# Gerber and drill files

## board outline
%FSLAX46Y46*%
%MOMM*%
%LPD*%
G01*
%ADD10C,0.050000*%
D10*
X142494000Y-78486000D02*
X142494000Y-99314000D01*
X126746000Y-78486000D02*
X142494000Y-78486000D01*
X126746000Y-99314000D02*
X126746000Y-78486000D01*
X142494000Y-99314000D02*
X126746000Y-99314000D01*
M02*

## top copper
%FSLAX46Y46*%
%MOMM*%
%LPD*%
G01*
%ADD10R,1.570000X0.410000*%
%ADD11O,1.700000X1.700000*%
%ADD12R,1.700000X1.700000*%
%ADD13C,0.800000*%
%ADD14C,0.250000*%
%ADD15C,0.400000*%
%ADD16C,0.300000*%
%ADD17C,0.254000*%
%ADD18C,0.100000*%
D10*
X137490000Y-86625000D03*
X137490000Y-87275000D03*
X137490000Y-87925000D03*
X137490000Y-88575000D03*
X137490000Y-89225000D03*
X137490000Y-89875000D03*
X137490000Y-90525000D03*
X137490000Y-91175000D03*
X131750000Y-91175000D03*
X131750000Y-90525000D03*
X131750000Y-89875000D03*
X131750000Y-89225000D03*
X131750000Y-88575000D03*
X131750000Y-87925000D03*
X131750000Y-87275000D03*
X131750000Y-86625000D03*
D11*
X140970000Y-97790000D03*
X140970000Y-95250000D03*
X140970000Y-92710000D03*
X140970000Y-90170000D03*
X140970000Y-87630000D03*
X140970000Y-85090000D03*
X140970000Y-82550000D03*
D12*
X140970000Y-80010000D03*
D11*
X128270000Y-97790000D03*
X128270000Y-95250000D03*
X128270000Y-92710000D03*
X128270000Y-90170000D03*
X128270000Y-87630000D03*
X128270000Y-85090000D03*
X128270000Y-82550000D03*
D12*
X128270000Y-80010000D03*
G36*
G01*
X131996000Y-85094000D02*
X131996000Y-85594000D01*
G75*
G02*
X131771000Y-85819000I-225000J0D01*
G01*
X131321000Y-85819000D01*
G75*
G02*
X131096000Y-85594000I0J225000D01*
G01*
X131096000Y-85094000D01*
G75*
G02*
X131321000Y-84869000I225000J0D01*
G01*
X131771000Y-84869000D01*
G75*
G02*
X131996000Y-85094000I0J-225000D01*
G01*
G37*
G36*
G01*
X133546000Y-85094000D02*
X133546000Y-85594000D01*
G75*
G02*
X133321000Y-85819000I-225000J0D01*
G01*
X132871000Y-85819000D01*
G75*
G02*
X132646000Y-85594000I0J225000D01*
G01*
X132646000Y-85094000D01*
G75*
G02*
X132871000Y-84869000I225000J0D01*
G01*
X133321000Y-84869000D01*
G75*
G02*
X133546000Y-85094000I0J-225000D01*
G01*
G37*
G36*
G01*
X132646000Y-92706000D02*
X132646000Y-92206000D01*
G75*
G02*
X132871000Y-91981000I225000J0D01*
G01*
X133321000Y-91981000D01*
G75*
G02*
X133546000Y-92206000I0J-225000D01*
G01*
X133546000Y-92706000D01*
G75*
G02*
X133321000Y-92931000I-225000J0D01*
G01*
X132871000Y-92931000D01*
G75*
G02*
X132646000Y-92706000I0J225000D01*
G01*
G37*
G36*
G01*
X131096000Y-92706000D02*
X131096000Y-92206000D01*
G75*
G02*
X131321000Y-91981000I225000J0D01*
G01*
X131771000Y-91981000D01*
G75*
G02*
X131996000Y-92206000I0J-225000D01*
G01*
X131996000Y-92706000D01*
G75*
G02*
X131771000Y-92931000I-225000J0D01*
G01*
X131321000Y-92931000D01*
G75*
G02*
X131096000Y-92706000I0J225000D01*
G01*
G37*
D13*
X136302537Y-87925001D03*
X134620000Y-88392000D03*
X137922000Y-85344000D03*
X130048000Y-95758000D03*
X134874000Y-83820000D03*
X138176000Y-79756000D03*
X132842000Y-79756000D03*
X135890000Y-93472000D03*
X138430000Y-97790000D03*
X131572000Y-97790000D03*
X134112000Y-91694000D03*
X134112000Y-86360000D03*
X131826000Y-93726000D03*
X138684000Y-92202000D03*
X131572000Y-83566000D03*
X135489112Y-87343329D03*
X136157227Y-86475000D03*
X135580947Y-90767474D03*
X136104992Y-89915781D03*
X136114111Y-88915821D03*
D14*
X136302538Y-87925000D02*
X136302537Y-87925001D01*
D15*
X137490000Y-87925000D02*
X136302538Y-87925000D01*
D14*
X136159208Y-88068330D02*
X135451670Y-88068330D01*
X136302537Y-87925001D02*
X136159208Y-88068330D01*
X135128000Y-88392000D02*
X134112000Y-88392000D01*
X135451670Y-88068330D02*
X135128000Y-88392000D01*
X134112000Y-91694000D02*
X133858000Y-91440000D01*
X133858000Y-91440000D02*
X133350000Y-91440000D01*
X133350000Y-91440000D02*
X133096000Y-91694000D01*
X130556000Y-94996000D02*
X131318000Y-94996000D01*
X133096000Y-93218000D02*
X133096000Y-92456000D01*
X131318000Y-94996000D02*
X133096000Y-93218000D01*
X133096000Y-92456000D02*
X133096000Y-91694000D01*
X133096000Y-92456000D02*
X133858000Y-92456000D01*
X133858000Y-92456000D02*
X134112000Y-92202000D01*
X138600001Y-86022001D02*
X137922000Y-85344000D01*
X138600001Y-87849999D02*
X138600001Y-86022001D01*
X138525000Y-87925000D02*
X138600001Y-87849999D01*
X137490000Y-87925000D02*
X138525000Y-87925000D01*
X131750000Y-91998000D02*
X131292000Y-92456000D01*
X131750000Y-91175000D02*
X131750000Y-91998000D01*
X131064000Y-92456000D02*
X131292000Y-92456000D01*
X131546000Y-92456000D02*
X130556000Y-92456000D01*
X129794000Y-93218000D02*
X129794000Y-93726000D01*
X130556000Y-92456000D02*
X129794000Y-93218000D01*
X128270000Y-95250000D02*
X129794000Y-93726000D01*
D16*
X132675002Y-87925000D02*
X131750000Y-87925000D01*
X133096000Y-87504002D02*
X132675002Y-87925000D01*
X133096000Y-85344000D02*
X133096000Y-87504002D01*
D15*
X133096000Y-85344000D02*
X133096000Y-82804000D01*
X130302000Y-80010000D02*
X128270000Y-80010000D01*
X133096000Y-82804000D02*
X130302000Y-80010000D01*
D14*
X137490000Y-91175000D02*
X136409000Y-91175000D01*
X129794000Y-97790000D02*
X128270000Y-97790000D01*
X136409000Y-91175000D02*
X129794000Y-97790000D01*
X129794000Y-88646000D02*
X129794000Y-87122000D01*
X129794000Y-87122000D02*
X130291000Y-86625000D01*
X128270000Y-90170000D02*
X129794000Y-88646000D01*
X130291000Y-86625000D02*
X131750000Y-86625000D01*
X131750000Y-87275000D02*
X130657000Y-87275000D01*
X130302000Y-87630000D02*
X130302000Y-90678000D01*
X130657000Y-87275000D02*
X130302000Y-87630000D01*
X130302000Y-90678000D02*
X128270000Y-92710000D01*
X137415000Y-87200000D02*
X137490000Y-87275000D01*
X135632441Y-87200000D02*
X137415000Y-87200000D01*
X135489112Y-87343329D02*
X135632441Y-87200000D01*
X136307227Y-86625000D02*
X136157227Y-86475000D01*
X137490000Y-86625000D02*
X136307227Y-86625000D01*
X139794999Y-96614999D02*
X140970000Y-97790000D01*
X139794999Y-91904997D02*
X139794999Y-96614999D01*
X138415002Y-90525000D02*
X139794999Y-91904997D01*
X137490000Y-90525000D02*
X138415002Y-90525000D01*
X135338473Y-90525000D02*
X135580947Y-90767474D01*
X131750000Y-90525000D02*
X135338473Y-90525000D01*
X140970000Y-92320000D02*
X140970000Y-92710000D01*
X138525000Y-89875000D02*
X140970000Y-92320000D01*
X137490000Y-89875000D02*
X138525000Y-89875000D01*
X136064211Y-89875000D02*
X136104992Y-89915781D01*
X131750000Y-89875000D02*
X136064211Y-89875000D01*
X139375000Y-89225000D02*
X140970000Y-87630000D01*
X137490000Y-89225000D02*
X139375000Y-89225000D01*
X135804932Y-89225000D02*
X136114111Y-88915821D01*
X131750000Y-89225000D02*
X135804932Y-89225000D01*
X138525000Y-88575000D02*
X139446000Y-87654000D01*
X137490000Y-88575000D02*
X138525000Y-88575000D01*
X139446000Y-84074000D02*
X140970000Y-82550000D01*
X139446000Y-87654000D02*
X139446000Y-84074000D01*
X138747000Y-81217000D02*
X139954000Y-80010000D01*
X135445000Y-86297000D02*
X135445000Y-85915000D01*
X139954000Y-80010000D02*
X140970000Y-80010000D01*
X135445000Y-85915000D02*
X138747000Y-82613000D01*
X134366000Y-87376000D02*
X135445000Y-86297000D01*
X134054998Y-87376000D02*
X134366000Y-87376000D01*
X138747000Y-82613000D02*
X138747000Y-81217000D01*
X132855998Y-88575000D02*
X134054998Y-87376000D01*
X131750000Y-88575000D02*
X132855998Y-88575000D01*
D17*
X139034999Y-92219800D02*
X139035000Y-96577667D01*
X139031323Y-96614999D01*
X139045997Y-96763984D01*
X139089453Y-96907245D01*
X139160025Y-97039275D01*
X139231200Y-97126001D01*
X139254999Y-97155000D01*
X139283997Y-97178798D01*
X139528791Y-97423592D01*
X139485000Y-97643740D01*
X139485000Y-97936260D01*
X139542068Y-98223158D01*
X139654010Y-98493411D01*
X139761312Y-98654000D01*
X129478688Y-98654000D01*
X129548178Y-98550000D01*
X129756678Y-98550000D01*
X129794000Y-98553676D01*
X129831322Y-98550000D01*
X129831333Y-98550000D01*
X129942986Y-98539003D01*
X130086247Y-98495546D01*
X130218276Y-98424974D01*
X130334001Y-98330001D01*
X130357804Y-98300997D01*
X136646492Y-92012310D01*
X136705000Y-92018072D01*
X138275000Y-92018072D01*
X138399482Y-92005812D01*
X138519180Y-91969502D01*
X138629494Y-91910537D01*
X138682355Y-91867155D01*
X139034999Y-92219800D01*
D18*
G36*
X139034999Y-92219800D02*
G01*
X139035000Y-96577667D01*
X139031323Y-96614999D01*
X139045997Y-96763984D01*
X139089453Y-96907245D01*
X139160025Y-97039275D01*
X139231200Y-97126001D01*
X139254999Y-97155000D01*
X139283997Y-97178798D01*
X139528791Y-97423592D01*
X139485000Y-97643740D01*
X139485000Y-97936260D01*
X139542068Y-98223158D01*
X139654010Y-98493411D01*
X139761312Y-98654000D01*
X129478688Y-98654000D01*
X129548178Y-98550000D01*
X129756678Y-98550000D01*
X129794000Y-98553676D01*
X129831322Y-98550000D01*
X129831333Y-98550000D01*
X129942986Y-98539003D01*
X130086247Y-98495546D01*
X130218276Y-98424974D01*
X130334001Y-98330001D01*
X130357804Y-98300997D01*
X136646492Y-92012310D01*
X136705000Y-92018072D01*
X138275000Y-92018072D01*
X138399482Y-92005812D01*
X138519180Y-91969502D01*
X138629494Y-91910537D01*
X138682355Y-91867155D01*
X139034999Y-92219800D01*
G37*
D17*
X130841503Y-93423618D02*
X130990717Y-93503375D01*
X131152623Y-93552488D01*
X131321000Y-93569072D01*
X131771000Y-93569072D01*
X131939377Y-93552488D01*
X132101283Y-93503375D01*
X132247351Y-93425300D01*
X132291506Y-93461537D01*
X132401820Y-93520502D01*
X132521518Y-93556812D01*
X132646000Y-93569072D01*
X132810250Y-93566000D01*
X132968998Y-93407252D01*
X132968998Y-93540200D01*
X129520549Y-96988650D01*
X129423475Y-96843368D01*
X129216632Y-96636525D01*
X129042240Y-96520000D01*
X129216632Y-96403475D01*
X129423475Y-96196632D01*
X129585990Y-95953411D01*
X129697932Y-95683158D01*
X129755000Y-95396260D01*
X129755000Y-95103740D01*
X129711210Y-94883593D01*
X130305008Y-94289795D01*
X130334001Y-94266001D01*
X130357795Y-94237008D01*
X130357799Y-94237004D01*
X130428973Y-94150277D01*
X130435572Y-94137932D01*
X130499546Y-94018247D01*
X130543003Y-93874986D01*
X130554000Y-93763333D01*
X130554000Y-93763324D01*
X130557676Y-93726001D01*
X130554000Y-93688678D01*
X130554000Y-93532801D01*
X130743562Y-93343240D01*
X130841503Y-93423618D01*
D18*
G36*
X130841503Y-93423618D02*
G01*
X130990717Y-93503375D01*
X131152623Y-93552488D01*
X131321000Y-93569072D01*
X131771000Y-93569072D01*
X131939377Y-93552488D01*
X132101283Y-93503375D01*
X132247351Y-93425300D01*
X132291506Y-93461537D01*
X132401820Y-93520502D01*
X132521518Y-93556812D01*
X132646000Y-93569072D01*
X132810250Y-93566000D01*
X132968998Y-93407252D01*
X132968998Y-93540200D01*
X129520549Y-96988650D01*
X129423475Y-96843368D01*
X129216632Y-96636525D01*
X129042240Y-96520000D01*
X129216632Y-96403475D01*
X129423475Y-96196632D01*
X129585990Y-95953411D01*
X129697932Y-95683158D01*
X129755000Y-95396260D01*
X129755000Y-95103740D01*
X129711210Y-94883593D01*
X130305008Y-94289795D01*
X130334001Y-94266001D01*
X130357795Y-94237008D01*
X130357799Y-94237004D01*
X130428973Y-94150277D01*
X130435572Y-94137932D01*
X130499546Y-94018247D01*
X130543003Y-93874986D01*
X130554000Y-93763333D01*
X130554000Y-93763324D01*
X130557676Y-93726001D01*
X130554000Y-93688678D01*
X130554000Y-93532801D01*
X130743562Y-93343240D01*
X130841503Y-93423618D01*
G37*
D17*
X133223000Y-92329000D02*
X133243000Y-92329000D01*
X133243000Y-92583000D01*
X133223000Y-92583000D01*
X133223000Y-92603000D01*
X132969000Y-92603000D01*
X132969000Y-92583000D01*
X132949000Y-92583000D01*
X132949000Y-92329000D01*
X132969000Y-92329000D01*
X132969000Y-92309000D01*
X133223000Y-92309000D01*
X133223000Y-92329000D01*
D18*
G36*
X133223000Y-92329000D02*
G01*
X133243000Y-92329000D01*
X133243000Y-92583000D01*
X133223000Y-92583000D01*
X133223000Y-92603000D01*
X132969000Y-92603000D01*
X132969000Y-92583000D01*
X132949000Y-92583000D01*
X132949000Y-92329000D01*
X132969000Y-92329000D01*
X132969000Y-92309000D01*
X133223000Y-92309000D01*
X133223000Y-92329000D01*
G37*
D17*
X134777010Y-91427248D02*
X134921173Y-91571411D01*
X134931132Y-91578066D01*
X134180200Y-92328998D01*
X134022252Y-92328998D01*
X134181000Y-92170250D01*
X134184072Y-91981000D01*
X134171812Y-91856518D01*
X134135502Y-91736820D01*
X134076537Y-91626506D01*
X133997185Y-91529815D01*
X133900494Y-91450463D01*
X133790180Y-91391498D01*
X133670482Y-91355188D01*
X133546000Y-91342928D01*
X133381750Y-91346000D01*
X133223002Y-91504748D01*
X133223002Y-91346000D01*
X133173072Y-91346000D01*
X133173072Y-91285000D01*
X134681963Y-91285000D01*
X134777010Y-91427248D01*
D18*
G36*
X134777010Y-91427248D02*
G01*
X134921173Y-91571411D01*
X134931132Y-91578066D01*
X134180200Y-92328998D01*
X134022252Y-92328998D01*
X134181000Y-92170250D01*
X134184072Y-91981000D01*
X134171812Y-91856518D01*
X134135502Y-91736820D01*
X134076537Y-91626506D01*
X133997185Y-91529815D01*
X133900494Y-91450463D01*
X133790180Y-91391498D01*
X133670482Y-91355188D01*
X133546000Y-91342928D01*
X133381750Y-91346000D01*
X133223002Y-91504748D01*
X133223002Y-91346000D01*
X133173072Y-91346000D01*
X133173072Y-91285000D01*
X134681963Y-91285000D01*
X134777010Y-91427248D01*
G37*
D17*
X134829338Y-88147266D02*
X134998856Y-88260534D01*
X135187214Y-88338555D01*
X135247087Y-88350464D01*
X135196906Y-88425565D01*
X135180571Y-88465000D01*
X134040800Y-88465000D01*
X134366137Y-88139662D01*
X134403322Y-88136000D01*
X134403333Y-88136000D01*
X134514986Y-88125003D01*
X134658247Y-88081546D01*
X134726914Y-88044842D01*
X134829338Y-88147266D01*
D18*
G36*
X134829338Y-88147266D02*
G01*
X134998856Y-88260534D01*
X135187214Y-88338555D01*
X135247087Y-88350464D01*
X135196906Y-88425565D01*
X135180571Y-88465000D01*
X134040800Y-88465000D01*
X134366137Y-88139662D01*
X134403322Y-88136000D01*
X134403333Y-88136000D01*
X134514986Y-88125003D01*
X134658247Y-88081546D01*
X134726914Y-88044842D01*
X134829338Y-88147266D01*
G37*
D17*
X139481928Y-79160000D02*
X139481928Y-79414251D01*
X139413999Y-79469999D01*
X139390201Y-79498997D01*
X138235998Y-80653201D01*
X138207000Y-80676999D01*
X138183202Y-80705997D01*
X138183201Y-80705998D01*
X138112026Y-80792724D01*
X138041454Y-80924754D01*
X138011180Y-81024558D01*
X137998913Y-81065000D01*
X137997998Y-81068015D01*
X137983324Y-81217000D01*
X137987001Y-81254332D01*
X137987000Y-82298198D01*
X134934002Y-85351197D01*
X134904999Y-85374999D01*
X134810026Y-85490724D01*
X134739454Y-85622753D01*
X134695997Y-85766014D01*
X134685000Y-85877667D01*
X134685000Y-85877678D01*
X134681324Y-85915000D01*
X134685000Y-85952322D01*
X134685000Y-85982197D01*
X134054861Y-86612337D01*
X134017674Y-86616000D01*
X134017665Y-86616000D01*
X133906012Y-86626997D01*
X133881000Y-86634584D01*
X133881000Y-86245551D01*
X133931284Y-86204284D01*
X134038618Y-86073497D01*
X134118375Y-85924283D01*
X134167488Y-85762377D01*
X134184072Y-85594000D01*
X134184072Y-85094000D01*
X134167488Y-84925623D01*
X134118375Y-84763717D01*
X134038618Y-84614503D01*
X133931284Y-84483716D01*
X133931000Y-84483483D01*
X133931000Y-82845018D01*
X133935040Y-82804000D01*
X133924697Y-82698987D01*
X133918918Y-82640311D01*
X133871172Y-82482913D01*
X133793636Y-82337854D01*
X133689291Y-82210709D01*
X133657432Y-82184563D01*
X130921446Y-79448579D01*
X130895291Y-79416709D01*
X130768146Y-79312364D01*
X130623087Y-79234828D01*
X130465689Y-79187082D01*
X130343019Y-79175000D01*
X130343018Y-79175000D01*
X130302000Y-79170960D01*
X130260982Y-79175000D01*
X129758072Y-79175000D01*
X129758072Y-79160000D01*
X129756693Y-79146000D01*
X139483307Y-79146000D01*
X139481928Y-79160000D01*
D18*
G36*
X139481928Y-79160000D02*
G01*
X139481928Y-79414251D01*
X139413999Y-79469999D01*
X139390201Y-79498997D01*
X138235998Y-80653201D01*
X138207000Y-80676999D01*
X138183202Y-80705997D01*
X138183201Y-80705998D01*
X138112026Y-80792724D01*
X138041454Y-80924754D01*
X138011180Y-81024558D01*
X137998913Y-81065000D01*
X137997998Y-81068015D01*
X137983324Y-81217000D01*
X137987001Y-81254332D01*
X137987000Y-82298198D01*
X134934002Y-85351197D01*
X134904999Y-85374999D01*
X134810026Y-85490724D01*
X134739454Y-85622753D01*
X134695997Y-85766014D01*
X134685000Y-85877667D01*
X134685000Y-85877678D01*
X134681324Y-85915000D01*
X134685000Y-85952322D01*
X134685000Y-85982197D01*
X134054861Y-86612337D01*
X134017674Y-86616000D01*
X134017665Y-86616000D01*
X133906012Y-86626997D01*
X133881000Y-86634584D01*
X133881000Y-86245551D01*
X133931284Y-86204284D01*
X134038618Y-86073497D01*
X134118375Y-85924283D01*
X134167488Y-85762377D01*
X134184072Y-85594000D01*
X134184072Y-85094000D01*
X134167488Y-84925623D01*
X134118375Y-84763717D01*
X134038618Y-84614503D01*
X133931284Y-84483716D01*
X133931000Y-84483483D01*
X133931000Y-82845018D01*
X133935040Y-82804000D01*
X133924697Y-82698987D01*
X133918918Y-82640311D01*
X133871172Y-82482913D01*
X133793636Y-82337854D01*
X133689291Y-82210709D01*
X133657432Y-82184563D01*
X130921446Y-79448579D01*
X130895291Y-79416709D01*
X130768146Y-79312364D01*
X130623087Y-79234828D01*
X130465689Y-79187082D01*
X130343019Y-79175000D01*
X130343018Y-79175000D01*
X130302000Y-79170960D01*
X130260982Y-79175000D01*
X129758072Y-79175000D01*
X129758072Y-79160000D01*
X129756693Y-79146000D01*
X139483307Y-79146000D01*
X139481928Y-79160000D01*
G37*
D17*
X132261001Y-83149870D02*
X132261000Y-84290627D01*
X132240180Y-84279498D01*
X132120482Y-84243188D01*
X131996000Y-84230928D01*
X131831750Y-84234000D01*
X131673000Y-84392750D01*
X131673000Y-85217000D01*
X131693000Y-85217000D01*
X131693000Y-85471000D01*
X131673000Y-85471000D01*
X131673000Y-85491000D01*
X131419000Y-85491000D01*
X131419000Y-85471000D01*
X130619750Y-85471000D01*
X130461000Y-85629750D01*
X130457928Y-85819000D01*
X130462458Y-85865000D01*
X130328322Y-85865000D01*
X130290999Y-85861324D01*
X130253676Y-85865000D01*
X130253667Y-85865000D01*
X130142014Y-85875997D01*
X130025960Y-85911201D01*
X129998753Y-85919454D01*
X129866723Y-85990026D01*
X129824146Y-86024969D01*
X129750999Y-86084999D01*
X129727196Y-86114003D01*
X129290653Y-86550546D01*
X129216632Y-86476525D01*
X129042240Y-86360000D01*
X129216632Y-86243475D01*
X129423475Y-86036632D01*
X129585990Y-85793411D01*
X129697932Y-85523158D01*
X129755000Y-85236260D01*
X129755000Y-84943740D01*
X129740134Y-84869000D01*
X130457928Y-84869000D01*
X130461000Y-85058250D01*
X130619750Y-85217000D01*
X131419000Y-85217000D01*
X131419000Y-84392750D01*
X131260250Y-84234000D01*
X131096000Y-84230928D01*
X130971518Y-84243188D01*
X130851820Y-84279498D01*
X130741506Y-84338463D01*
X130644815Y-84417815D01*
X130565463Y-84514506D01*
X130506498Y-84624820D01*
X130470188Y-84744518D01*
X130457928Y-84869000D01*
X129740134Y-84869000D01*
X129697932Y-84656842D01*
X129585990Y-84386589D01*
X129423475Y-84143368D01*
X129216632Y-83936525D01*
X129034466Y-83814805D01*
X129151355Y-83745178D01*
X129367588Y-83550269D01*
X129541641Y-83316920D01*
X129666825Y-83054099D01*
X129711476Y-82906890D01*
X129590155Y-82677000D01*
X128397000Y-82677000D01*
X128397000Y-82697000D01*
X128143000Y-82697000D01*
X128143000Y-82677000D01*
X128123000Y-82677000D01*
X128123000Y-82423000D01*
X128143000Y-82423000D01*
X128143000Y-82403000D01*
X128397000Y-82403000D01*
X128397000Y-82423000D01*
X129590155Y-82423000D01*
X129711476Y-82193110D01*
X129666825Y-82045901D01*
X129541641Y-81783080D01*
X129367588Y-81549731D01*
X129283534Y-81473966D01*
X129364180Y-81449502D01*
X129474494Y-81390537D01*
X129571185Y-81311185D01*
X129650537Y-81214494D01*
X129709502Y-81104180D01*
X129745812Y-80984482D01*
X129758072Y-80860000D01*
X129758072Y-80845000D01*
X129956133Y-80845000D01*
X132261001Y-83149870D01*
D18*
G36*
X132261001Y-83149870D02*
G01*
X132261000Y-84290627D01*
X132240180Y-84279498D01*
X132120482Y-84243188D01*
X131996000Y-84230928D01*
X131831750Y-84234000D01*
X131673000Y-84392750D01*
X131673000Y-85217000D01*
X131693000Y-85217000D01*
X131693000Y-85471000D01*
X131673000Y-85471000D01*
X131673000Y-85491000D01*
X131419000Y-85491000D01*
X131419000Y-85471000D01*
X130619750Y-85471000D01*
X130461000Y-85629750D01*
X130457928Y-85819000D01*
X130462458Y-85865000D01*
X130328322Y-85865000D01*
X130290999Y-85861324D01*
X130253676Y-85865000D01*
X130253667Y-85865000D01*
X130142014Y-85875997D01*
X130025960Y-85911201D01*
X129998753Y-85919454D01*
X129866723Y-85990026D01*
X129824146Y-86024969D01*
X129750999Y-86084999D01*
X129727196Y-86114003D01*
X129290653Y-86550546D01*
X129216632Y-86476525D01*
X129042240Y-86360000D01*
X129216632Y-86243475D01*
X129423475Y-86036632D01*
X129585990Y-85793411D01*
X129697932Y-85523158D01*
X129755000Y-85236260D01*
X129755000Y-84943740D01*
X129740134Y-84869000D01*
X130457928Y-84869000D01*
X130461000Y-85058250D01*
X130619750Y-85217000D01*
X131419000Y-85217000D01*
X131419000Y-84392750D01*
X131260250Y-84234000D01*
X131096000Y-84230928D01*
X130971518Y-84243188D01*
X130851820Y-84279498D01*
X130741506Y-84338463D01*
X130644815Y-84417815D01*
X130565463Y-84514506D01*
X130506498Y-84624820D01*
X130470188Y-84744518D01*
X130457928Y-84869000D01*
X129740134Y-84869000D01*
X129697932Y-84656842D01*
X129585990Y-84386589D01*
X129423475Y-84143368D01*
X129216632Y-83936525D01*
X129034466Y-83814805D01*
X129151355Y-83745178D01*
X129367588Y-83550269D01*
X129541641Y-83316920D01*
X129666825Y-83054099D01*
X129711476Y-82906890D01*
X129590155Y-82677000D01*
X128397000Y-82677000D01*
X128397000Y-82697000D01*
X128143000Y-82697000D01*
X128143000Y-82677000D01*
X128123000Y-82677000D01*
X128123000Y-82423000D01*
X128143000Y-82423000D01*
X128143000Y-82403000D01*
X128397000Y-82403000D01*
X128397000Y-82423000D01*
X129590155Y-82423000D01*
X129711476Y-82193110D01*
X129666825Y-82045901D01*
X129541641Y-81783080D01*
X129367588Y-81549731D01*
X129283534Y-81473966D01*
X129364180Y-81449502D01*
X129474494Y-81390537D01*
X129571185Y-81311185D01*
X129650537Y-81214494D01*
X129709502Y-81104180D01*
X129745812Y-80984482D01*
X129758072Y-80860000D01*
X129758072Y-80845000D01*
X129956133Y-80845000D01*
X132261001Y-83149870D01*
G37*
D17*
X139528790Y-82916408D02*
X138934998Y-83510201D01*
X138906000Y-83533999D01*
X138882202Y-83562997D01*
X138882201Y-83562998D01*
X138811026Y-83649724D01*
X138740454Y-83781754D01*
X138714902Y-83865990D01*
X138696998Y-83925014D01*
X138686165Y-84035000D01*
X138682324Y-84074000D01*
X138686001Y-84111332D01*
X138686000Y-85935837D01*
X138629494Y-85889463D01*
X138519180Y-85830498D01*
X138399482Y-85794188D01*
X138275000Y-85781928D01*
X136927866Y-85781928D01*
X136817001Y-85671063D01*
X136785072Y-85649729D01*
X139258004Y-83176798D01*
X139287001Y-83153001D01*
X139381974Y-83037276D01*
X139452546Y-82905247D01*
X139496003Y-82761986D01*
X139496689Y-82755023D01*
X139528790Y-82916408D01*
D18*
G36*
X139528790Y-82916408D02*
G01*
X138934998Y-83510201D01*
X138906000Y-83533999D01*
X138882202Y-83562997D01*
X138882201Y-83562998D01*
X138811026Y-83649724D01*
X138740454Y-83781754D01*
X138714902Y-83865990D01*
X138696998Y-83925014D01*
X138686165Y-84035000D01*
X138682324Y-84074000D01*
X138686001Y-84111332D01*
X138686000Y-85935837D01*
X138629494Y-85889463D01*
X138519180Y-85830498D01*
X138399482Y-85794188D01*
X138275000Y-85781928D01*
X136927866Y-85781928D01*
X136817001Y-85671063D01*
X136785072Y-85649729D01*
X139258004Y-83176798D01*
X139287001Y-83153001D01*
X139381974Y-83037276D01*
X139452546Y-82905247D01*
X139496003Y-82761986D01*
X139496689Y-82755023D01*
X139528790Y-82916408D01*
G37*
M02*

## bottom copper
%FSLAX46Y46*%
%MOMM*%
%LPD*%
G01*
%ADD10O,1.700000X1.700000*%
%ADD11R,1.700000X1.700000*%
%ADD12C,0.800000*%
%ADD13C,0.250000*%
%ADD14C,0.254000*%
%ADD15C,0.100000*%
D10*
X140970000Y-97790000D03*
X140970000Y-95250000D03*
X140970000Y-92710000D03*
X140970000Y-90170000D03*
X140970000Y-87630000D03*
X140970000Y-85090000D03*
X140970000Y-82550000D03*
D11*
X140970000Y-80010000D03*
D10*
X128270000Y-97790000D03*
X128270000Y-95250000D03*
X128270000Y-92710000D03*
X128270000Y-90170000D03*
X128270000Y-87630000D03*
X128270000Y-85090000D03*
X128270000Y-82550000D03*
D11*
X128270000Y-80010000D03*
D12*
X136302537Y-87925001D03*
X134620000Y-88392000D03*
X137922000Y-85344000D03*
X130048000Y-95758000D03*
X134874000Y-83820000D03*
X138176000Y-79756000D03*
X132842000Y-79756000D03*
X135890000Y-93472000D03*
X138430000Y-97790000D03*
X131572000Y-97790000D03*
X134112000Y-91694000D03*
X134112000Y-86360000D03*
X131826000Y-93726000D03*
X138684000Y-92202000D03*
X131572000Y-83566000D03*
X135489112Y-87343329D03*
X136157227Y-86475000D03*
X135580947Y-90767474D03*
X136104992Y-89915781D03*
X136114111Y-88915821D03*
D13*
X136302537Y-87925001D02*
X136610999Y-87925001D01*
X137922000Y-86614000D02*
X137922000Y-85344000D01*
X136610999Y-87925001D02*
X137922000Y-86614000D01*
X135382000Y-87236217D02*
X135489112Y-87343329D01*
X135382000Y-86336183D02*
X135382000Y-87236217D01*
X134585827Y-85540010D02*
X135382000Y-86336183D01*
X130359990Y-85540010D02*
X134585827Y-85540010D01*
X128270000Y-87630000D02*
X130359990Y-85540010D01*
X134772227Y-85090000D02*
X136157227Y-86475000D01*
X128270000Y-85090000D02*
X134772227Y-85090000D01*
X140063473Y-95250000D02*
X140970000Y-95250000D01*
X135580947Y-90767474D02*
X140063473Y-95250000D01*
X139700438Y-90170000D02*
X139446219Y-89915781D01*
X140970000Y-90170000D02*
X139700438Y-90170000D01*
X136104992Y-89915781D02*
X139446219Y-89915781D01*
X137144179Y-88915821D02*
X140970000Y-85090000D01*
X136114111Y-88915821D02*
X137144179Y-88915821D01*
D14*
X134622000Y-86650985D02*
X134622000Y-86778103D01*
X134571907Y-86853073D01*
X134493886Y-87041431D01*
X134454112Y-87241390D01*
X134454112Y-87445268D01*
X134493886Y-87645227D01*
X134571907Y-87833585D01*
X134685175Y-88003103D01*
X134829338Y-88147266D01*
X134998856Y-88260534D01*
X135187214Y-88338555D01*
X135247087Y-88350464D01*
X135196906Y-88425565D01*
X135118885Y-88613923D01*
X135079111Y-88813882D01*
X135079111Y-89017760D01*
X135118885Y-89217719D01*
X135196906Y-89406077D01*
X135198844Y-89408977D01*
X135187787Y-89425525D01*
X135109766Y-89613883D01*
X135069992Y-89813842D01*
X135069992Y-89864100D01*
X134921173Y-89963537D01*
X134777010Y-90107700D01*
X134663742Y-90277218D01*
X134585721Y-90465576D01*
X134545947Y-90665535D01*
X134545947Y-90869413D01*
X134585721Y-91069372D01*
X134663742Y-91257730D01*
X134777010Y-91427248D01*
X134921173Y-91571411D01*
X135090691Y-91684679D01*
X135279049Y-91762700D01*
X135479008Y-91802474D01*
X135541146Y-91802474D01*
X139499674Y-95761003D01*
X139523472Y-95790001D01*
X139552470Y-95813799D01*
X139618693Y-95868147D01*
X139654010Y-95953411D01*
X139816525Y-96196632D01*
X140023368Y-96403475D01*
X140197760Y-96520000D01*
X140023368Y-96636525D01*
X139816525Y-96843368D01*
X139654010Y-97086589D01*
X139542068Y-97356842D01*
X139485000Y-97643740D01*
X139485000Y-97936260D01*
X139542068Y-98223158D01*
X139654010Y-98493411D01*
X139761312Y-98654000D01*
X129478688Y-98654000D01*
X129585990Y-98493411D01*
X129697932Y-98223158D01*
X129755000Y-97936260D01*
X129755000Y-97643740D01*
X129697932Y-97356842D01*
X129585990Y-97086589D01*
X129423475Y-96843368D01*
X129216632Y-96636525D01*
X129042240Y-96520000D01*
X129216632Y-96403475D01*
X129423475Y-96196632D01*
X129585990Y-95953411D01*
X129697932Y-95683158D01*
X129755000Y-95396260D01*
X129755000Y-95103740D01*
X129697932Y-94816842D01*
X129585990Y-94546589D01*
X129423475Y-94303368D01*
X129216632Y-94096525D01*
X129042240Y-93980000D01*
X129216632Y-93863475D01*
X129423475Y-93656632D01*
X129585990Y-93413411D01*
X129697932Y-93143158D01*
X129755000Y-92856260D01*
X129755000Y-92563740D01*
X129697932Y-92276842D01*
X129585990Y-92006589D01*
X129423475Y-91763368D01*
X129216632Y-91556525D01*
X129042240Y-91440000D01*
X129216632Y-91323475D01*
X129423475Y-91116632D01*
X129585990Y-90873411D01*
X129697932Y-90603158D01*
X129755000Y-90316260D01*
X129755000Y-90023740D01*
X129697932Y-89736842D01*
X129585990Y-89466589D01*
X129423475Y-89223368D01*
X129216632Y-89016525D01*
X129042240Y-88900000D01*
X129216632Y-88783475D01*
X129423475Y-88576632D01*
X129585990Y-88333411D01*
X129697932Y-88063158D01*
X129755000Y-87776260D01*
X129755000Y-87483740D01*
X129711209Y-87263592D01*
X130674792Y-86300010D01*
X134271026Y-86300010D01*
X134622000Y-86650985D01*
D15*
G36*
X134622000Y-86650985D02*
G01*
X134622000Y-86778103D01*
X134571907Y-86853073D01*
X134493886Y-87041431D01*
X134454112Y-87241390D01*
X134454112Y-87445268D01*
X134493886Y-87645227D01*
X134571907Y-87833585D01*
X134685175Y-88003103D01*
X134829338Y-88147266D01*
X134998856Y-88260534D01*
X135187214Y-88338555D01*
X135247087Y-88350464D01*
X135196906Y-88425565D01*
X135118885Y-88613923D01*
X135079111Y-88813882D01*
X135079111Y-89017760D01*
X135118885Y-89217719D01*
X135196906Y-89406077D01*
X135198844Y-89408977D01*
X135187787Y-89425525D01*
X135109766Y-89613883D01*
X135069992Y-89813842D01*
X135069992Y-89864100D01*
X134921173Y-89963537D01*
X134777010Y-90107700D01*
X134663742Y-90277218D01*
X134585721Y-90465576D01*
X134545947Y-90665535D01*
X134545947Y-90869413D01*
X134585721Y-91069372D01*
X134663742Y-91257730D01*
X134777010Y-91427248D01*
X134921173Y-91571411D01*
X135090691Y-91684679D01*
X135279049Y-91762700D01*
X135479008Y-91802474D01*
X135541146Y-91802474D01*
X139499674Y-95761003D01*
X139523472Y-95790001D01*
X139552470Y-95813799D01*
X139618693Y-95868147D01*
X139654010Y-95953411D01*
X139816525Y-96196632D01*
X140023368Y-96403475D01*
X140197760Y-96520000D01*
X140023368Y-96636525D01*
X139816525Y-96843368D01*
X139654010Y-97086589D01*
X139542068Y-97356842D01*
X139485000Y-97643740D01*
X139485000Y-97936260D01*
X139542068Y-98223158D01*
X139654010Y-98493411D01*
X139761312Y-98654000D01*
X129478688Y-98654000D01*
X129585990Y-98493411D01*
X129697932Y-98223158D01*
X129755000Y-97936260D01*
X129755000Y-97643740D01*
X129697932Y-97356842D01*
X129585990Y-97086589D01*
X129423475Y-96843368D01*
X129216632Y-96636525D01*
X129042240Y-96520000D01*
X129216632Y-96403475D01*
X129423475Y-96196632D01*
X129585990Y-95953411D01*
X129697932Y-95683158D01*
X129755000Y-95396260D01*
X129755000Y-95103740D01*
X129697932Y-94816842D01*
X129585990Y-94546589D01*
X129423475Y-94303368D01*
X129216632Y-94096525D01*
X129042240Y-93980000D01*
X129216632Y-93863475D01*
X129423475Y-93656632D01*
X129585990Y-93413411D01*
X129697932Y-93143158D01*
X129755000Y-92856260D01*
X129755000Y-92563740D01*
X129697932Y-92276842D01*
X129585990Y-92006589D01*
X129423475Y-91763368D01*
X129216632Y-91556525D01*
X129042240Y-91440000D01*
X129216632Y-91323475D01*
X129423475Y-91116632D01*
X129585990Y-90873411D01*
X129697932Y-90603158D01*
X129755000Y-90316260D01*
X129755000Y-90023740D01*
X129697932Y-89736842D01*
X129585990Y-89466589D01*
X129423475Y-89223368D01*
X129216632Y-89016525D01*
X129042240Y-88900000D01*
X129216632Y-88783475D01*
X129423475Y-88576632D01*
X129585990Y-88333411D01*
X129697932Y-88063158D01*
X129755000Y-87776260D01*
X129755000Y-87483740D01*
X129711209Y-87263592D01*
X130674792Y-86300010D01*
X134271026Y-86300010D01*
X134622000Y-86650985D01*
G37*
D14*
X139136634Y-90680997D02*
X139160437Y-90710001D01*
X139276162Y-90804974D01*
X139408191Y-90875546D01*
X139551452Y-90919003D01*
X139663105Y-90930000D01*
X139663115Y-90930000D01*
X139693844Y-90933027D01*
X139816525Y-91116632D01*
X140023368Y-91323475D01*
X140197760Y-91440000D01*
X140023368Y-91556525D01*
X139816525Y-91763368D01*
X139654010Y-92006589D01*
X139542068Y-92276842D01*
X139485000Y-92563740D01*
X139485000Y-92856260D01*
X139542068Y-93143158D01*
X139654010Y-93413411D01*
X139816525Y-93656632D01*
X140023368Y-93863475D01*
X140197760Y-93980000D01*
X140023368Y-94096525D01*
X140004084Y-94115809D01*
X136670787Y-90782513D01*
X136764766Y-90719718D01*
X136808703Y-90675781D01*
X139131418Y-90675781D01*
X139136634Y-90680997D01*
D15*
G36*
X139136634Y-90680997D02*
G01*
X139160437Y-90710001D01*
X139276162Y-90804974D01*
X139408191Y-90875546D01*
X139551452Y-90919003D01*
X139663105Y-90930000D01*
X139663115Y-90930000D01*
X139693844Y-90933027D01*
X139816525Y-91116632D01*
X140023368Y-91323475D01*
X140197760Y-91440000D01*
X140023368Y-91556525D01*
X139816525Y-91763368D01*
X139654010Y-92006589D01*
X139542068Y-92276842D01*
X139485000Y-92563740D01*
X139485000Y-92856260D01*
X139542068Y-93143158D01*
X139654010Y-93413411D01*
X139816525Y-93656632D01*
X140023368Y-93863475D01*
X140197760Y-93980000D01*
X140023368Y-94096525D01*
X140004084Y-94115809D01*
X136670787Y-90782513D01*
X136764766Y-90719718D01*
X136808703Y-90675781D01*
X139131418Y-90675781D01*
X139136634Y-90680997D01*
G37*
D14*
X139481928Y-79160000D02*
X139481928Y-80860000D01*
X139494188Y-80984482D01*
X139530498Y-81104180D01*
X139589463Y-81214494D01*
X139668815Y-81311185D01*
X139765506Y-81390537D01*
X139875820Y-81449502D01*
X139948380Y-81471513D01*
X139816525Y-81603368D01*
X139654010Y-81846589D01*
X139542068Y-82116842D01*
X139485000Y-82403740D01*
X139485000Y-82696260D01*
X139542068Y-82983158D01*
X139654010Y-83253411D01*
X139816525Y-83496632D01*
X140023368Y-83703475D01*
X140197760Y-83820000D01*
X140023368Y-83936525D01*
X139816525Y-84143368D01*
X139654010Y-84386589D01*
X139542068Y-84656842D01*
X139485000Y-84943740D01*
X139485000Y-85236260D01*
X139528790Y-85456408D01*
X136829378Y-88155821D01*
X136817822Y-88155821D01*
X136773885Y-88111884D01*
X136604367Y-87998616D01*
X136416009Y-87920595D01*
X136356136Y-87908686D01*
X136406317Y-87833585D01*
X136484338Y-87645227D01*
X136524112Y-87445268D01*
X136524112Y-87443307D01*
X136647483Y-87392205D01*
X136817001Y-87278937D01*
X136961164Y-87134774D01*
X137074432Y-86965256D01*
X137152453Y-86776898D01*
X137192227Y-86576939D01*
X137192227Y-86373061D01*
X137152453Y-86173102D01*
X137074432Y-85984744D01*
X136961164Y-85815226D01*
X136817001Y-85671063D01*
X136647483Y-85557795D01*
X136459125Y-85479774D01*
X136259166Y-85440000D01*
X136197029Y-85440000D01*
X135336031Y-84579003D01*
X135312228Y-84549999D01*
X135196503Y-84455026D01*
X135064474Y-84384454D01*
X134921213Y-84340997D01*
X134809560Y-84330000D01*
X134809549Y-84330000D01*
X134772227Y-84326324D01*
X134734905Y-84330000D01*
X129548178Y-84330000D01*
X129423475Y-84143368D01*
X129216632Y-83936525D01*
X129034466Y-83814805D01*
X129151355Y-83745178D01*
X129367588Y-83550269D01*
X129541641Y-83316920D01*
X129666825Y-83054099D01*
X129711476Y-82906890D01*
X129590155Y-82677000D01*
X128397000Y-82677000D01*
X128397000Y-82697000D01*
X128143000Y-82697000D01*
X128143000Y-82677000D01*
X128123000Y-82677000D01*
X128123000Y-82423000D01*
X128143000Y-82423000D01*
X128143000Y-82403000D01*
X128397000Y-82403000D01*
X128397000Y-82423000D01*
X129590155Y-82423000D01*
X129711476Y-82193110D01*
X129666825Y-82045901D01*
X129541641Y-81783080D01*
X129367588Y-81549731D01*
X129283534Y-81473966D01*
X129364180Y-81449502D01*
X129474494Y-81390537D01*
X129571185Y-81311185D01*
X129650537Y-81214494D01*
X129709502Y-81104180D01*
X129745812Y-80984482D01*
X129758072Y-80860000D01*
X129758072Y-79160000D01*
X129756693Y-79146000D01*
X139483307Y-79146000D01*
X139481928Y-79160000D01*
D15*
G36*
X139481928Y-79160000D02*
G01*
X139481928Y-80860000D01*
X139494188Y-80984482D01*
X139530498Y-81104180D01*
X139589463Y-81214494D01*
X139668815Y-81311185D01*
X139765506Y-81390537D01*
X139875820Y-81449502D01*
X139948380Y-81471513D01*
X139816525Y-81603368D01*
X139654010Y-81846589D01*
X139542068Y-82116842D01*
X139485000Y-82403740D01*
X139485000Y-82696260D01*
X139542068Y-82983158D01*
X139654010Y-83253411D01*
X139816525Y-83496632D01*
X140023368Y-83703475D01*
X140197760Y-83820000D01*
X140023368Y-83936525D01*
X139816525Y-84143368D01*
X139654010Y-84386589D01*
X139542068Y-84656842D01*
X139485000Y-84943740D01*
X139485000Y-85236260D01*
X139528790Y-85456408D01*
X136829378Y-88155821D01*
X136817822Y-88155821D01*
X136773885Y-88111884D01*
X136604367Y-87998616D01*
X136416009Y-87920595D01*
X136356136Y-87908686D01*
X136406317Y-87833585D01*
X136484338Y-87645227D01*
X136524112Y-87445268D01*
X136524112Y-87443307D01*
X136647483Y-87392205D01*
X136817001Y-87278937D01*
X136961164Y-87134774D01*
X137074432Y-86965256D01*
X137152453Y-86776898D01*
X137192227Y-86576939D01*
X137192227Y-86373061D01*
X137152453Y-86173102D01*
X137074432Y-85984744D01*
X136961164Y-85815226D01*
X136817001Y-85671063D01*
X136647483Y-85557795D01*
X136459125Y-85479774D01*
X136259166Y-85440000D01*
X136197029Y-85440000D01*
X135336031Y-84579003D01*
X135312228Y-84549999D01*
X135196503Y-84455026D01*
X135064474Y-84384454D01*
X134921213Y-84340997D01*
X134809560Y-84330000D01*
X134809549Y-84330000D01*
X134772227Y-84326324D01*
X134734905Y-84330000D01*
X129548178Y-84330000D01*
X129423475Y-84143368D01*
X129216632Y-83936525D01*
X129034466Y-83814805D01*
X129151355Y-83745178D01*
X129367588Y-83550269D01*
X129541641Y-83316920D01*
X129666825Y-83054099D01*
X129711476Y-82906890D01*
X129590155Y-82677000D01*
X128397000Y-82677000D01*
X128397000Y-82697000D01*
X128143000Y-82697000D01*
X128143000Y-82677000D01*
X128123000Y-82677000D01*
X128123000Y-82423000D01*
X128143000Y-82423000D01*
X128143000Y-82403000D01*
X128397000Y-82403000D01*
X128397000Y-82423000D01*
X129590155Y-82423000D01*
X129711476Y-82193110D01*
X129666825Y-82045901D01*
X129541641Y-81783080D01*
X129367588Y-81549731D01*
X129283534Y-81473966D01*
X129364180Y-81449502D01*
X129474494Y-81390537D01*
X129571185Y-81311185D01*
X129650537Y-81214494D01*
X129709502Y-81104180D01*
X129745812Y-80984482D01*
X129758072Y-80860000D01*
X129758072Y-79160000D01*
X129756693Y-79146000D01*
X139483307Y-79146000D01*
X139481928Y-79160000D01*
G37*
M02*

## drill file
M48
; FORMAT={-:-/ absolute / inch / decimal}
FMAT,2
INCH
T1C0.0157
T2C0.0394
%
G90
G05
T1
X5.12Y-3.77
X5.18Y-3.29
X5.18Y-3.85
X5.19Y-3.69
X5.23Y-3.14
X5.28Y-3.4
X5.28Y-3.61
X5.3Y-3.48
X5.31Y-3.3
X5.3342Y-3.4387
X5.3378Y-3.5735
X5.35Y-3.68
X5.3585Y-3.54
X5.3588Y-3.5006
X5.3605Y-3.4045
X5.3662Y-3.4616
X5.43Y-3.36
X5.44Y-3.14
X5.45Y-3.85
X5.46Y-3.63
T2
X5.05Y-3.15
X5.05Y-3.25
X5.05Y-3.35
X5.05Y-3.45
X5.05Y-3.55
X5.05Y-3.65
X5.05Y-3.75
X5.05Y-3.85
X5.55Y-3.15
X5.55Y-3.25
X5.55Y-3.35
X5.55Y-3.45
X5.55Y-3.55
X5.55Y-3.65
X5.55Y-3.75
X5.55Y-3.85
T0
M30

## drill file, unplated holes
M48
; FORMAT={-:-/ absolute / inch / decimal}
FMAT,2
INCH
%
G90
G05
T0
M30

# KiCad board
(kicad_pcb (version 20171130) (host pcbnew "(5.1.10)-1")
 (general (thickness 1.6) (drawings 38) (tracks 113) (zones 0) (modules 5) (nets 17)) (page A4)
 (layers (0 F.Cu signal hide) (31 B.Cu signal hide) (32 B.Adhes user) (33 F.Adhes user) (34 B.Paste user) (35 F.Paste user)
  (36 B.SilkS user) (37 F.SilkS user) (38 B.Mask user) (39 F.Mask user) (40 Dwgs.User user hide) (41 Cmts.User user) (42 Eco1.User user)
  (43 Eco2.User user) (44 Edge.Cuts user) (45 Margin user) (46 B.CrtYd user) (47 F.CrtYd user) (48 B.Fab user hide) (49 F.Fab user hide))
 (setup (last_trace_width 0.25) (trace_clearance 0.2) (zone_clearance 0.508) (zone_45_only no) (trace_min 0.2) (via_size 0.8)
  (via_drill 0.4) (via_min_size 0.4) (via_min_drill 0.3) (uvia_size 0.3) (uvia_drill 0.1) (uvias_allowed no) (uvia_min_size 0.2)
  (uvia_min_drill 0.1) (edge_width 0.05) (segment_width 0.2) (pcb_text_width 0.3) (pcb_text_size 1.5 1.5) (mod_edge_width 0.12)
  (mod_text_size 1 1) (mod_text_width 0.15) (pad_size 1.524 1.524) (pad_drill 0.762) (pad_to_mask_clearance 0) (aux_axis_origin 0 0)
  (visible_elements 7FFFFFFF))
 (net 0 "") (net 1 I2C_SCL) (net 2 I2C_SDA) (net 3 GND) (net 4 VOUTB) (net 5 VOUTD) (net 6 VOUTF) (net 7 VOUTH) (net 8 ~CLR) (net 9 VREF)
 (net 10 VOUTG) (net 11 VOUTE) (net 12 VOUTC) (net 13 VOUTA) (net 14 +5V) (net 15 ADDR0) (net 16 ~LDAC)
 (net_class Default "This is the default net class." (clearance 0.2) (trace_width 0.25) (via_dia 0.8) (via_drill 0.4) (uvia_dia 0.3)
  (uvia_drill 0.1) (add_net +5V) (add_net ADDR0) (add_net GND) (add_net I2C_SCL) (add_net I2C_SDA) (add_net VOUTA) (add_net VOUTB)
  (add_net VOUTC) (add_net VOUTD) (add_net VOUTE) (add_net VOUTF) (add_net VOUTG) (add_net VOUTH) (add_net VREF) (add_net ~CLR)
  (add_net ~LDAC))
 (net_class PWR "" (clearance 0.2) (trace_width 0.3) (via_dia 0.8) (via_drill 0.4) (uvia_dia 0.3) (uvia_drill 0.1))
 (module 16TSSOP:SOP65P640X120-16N (layer F.Cu) (at 134.62 88.9)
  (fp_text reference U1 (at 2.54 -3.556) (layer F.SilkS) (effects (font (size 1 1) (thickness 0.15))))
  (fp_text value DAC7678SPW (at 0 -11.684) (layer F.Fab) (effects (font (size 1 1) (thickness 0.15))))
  (pad 16 smd rect (at 2.87 -2.275) (size 1.57 0.41) (layers F.Cu F.Paste F.Mask) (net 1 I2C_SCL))
  (pad 15 smd rect (at 2.87 -1.625) (size 1.57 0.41) (layers F.Cu F.Paste F.Mask) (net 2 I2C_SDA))
  (pad 14 smd rect (at 2.87 -0.975) (size 1.57 0.41) (layers F.Cu F.Paste F.Mask) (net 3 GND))
  (pad 13 smd rect (at 2.87 -0.325) (size 1.57 0.41) (layers F.Cu F.Paste F.Mask) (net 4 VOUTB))
  (pad 12 smd rect (at 2.87 0.325) (size 1.57 0.41) (layers F.Cu F.Paste F.Mask) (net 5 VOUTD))
  (pad 11 smd rect (at 2.87 0.975) (size 1.57 0.41) (layers F.Cu F.Paste F.Mask) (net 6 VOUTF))
  (pad 10 smd rect (at 2.87 1.625) (size 1.57 0.41) (layers F.Cu F.Paste F.Mask) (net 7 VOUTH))
  (pad 9 smd rect (at 2.87 2.275) (size 1.57 0.41) (layers F.Cu F.Paste F.Mask) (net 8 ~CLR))
  (pad 8 smd rect (at -2.87 2.275) (size 1.57 0.41) (layers F.Cu F.Paste F.Mask) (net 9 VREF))
  (pad 7 smd rect (at -2.87 1.625) (size 1.57 0.41) (layers F.Cu F.Paste F.Mask) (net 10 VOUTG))
  (pad 6 smd rect (at -2.87 0.975) (size 1.57 0.41) (layers F.Cu F.Paste F.Mask) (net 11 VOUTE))
  (pad 5 smd rect (at -2.87 0.325) (size 1.57 0.41) (layers F.Cu F.Paste F.Mask) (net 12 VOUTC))
  (pad 4 smd rect (at -2.87 -0.325) (size 1.57 0.41) (layers F.Cu F.Paste F.Mask) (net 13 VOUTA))
  (pad 3 smd rect (at -2.87 -0.975) (size 1.57 0.41) (layers F.Cu F.Paste F.Mask) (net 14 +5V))
  (pad 2 smd rect (at -2.87 -1.625) (size 1.57 0.41) (layers F.Cu F.Paste F.Mask) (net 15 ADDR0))
  (pad 1 smd rect (at -2.87 -2.275) (size 1.57 0.41) (layers F.Cu F.Paste F.Mask) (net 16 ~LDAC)))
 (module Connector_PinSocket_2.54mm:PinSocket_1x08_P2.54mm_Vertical (layer B.Cu) (at 140.97 80.01 180)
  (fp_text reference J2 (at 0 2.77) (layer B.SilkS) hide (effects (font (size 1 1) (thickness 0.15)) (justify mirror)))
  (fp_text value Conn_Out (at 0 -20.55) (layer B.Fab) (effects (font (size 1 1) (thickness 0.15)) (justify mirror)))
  (pad 8 thru_hole oval (at 0 -17.78 180) (size 1.7 1.7) (drill 1) (layers *.Cu *.Mask) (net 7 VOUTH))
  (pad 7 thru_hole oval (at 0 -15.24 180) (size 1.7 1.7) (drill 1) (layers *.Cu *.Mask) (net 10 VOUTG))
  (pad 6 thru_hole oval (at 0 -12.7 180) (size 1.7 1.7) (drill 1) (layers *.Cu *.Mask) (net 6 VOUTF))
  (pad 5 thru_hole oval (at 0 -10.16 180) (size 1.7 1.7) (drill 1) (layers *.Cu *.Mask) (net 11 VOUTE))
  (pad 4 thru_hole oval (at 0 -7.62 180) (size 1.7 1.7) (drill 1) (layers *.Cu *.Mask) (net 5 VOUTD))
  (pad 3 thru_hole oval (at 0 -5.08 180) (size 1.7 1.7) (drill 1) (layers *.Cu *.Mask) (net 12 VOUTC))
  (pad 2 thru_hole oval (at 0 -2.54 180) (size 1.7 1.7) (drill 1) (layers *.Cu *.Mask) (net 4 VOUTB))
  (pad 1 thru_hole rect (at 0 0 180) (size 1.7 1.7) (drill 1) (layers *.Cu *.Mask) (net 13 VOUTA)))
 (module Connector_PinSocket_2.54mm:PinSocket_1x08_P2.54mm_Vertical (layer B.Cu) (at 128.27 80.01 180)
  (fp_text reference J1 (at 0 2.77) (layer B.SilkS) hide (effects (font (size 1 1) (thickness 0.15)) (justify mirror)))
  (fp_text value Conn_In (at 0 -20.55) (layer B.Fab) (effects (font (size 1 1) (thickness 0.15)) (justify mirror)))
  (pad 8 thru_hole oval (at 0 -17.78 180) (size 1.7 1.7) (drill 1) (layers *.Cu *.Mask) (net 8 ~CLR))
  (pad 7 thru_hole oval (at 0 -15.24 180) (size 1.7 1.7) (drill 1) (layers *.Cu *.Mask) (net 9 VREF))
  (pad 6 thru_hole oval (at 0 -12.7 180) (size 1.7 1.7) (drill 1) (layers *.Cu *.Mask) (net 15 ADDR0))
  (pad 5 thru_hole oval (at 0 -10.16 180) (size 1.7 1.7) (drill 1) (layers *.Cu *.Mask) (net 16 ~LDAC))
  (pad 4 thru_hole oval (at 0 -7.62 180) (size 1.7 1.7) (drill 1) (layers *.Cu *.Mask) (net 2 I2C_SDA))
  (pad 3 thru_hole oval (at 0 -5.08 180) (size 1.7 1.7) (drill 1) (layers *.Cu *.Mask) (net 1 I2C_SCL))
  (pad 2 thru_hole oval (at 0 -2.54 180) (size 1.7 1.7) (drill 1) (layers *.Cu *.Mask) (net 3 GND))
  (pad 1 thru_hole rect (at 0 0 180) (size 1.7 1.7) (drill 1) (layers *.Cu *.Mask) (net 14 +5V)))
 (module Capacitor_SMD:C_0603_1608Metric (layer F.Cu) (at 132.321 85.344 180)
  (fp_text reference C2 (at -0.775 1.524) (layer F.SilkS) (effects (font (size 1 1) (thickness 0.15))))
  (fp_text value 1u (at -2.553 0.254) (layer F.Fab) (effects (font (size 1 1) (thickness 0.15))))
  (pad 2 smd roundrect (at 0.775 0 180) (size 0.9 0.95) (layers F.Cu F.Paste F.Mask) (roundrect_rratio 0.25) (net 3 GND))
  (pad 1 smd roundrect (at -0.775 0 180) (size 0.9 0.95) (layers F.Cu F.Paste F.Mask) (roundrect_rratio 0.25) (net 14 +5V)))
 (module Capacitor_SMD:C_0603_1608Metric (layer F.Cu) (at 132.321 92.456)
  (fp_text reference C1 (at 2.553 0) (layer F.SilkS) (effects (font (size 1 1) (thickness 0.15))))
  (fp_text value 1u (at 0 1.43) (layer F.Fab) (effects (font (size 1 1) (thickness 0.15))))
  (pad 2 smd roundrect (at 0.775 0) (size 0.9 0.95) (layers F.Cu F.Paste F.Mask) (roundrect_rratio 0.25) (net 3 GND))
  (pad 1 smd roundrect (at -0.775 0) (size 0.9 0.95) (layers F.Cu F.Paste F.Mask) (roundrect_rratio 0.25) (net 9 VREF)))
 (gr_line (start 142.494 78.486) (end 142.494 99.314) (layer Edge.Cuts) (width 0.05))
 (gr_line (start 126.746 78.486) (end 142.494 78.486) (layer Edge.Cuts) (width 0.05))
 (gr_line (start 126.746 99.314) (end 126.746 78.486) (layer Edge.Cuts) (width 0.05))
 (gr_line (start 142.494 99.314) (end 126.746 99.314) (layer Edge.Cuts) (width 0.05))
 (via (at 136.302537 87.925001) (size 0.8) (drill 0.4) (layers F.Cu B.Cu) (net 3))
 (segment (start 136.302538 87.925) (end 136.302537 87.925001) (width 0.25) (layer F.Cu) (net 3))
 (segment (start 137.49 87.925) (end 136.302538 87.925) (width 0.4) (layer F.Cu) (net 3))
 (via (at 134.62 88.392) (size 0.8) (drill 0.4) (layers F.Cu B.Cu) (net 3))
 (segment (start 136.159208 88.06833) (end 135.45167 88.06833) (width 0.25) (layer F.Cu) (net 3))
 (segment (start 136.302537 87.925001) (end 136.159208 88.06833) (width 0.25) (layer F.Cu) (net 3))
 (segment (start 135.128 88.392) (end 134.112 88.392) (width 0.25) (layer F.Cu) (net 3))
 (segment (start 135.45167 88.06833) (end 135.128 88.392) (width 0.25) (layer F.Cu) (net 3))
 (segment (start 136.302537 87.925001) (end 136.610999 87.925001) (width 0.25) (layer B.Cu) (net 3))
 (via (at 137.922 85.344) (size 0.8) (drill 0.4) (layers F.Cu B.Cu) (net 3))
 (segment (start 137.922 86.614) (end 137.922 85.344) (width 0.25) (layer B.Cu) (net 3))
 (segment (start 136.610999 87.925001) (end 137.922 86.614) (width 0.25) (layer B.Cu) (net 3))
 (via (at 130.048 95.758) (size 0.8) (drill 0.4) (layers F.Cu B.Cu) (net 3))
 (via (at 134.874 83.82) (size 0.8) (drill 0.4) (layers F.Cu B.Cu) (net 3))
 (via (at 138.176 79.756) (size 0.8) (drill 0.4) (layers F.Cu B.Cu) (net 3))
 (via (at 132.842 79.756) (size 0.8) (drill 0.4) (layers F.Cu B.Cu) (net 3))
 (via (at 135.89 93.472) (size 0.8) (drill 0.4) (layers F.Cu B.Cu) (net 3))
 (via (at 138.43 97.79) (size 0.8) (drill 0.4) (layers F.Cu B.Cu) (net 3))
 (via (at 131.572 97.79) (size 0.8) (drill 0.4) (layers F.Cu B.Cu) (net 3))
 (via (at 134.112 91.694) (size 0.8) (drill 0.4) (layers F.Cu B.Cu) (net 3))
 (via (at 134.112 86.36) (size 0.8) (drill 0.4) (layers F.Cu B.Cu) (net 3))
 (segment (start 134.112 91.694) (end 133.858 91.44) (width 0.25) (layer F.Cu) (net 3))
 (segment (start 133.858 91.44) (end 133.35 91.44) (width 0.25) (layer F.Cu) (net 3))
 (segment (start 133.35 91.44) (end 133.096 91.694) (width 0.25) (layer F.Cu) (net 3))
 (segment (start 130.556 94.996) (end 131.318 94.996) (width 0.25) (layer F.Cu) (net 3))
 (segment (start 133.096 93.218) (end 133.096 92.456) (width 0.25) (layer F.Cu) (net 3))
 (segment (start 131.318 94.996) (end 133.096 93.218) (width 0.25) (layer F.Cu) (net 3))
 (segment (start 133.096 92.456) (end 133.096 91.694) (width 0.25) (layer F.Cu) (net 3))
 (segment (start 133.096 92.456) (end 133.858 92.456) (width 0.25) (layer F.Cu) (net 3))
 (segment (start 133.858 92.456) (end 134.112 92.202) (width 0.25) (layer F.Cu) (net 3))
 (via (at 131.826 93.726) (size 0.8) (drill 0.4) (layers F.Cu B.Cu) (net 3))
 (via (at 138.684 92.202) (size 0.8) (drill 0.4) (layers F.Cu B.Cu) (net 3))
 (segment (start 138.600001 86.022001) (end 137.922 85.344) (width 0.25) (layer F.Cu) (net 3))
 (segment (start 138.600001 87.849999) (end 138.600001 86.022001) (width 0.25) (layer F.Cu) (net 3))
 (segment (start 138.525 87.925) (end 138.600001 87.849999) (width 0.25) (layer F.Cu) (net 3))
 (segment (start 137.49 87.925) (end 138.525 87.925) (width 0.25) (layer F.Cu) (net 3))
 (via (at 131.572 83.566) (size 0.8) (drill 0.4) (layers F.Cu B.Cu) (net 3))
 (segment (start 131.75 91.998) (end 131.292 92.456) (width 0.25) (layer F.Cu) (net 9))
 (segment (start 131.75 91.175) (end 131.75 91.998) (width 0.25) (layer F.Cu) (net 9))
 (segment (start 131.064 92.456) (end 131.292 92.456) (width 0.25) (layer F.Cu) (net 9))
 (segment (start 131.546 92.456) (end 130.556 92.456) (width 0.25) (layer F.Cu) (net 9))
 (segment (start 129.794 93.218) (end 129.794 93.726) (width 0.25) (layer F.Cu) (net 9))
 (segment (start 130.556 92.456) (end 129.794 93.218) (width 0.25) (layer F.Cu) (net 9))
 (segment (start 128.27 95.25) (end 129.794 93.726) (width 0.25) (layer F.Cu) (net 9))
 (segment (start 132.675002 87.925) (end 131.75 87.925) (width 0.3) (layer F.Cu) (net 14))
 (segment (start 133.096 87.504002) (end 132.675002 87.925) (width 0.3) (layer F.Cu) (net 14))
 (segment (start 133.096 85.344) (end 133.096 87.504002) (width 0.3) (layer F.Cu) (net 14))
 (segment (start 133.096 85.344) (end 133.096 82.804) (width 0.4) (layer F.Cu) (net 14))
 (segment (start 130.302 80.01) (end 128.27 80.01) (width 0.4) (layer F.Cu) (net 14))
 (segment (start 133.096 82.804) (end 130.302 80.01) (width 0.4) (layer F.Cu) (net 14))
 (segment (start 137.49 91.175) (end 136.409 91.175) (width 0.25) (layer F.Cu) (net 8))
 (segment (start 129.794 97.79) (end 128.27 97.79) (width 0.25) (layer F.Cu) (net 8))
 (segment (start 136.409 91.175) (end 129.794 97.79) (width 0.25) (layer F.Cu) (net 8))
 (segment (start 129.794 88.646) (end 129.794 87.122) (width 0.25) (layer F.Cu) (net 16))
 (segment (start 129.794 87.122) (end 130.291 86.625) (width 0.25) (layer F.Cu) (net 16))
 (segment (start 128.27 90.17) (end 129.794 88.646) (width 0.25) (layer F.Cu) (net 16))
 (segment (start 130.291 86.625) (end 131.75 86.625) (width 0.25) (layer F.Cu) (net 16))
 (segment (start 131.75 87.275) (end 130.657 87.275) (width 0.25) (layer F.Cu) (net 15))
 (segment (start 130.302 87.63) (end 130.302 90.678) (width 0.25) (layer F.Cu) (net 15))
 (segment (start 130.657 87.275) (end 130.302 87.63) (width 0.25) (layer F.Cu) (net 15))
 (segment (start 130.302 90.678) (end 128.27 92.71) (width 0.25) (layer F.Cu) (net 15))
 (via (at 135.489112 87.343329) (size 0.8) (drill 0.4) (layers F.Cu B.Cu) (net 2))
 (segment (start 137.415 87.2) (end 137.49 87.275) (width 0.25) (layer F.Cu) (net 2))
 (segment (start 135.632441 87.2) (end 137.415 87.2) (width 0.25) (layer F.Cu) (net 2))
 (segment (start 135.489112 87.343329) (end 135.632441 87.2) (width 0.25) (layer F.Cu) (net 2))
 (segment (start 135.382 87.236217) (end 135.489112 87.343329) (width 0.25) (layer B.Cu) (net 2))
 (segment (start 135.382 86.336183) (end 135.382 87.236217) (width 0.25) (layer B.Cu) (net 2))
 (segment (start 134.585827 85.54001) (end 135.382 86.336183) (width 0.25) (layer B.Cu) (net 2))
 (segment (start 130.35999 85.54001) (end 134.585827 85.54001) (width 0.25) (layer B.Cu) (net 2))
 (segment (start 128.27 87.63) (end 130.35999 85.54001) (width 0.25) (layer B.Cu) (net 2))
 (segment (start 134.772227 85.09) (end 136.157227 86.475) (width 0.25) (layer B.Cu) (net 1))
 (via (at 136.157227 86.475) (size 0.8) (drill 0.4) (layers F.Cu B.Cu) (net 1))
 (segment (start 128.27 85.09) (end 134.772227 85.09) (width 0.25) (layer B.Cu) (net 1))
 (segment (start 136.307227 86.625) (end 136.157227 86.475) (width 0.25) (layer F.Cu) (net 1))
 (segment (start 137.49 86.625) (end 136.307227 86.625) (width 0.25) (layer F.Cu) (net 1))
 (segment (start 139.794999 96.614999) (end 140.97 97.79) (width 0.25) (layer F.Cu) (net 7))
 (segment (start 139.794999 91.904997) (end 139.794999 96.614999) (width 0.25) (layer F.Cu) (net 7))
 (segment (start 138.415002 90.525) (end 139.794999 91.904997) (width 0.25) (layer F.Cu) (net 7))
 (segment (start 137.49 90.525) (end 138.415002 90.525) (width 0.25) (layer F.Cu) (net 7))
 (via (at 135.580947 90.767474) (size 0.8) (drill 0.4) (layers F.Cu B.Cu) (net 10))
 (segment (start 135.338473 90.525) (end 135.580947 90.767474) (width 0.25) (layer F.Cu) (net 10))
 (segment (start 131.75 90.525) (end 135.338473 90.525) (width 0.25) (layer F.Cu) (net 10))
 (segment (start 140.063473 95.25) (end 140.97 95.25) (width 0.25) (layer B.Cu) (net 10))
 (segment (start 135.580947 90.767474) (end 140.063473 95.25) (width 0.25) (layer B.Cu) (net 10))
 (segment (start 140.97 92.32) (end 140.97 92.71) (width 0.25) (layer F.Cu) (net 6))
 (segment (start 138.525 89.875) (end 140.97 92.32) (width 0.25) (layer F.Cu) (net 6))
 (segment (start 137.49 89.875) (end 138.525 89.875) (width 0.25) (layer F.Cu) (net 6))
 (via (at 136.104992 89.915781) (size 0.8) (drill 0.4) (layers F.Cu B.Cu) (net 11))
 (segment (start 136.064211 89.875) (end 136.104992 89.915781) (width 0.25) (layer F.Cu) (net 11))
 (segment (start 131.75 89.875) (end 136.064211 89.875) (width 0.25) (layer F.Cu) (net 11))
 (segment (start 139.700438 90.17) (end 139.446219 89.915781) (width 0.25) (layer B.Cu) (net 11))
 (segment (start 140.97 90.17) (end 139.700438 90.17) (width 0.25) (layer B.Cu) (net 11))
 (segment (start 136.104992 89.915781) (end 139.446219 89.915781) (width 0.25) (layer B.Cu) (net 11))
 (segment (start 139.375 89.225) (end 140.97 87.63) (width 0.25) (layer F.Cu) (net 5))
 (segment (start 137.49 89.225) (end 139.375 89.225) (width 0.25) (layer F.Cu) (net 5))
 (via (at 136.114111 88.915821) (size 0.8) (drill 0.4) (layers F.Cu B.Cu) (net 12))
 (segment (start 135.804932 89.225) (end 136.114111 88.915821) (width 0.25) (layer F.Cu) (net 12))
 (segment (start 131.75 89.225) (end 135.804932 89.225) (width 0.25) (layer F.Cu) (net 12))
 (segment (start 137.144179 88.915821) (end 140.97 85.09) (width 0.25) (layer B.Cu) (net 12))
 (segment (start 136.114111 88.915821) (end 137.144179 88.915821) (width 0.25) (layer B.Cu) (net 12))
 (segment (start 138.525 88.575) (end 139.446 87.654) (width 0.25) (layer F.Cu) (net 4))
 (segment (start 137.49 88.575) (end 138.525 88.575) (width 0.25) (layer F.Cu) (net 4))
 (segment (start 139.446 84.074) (end 140.97 82.55) (width 0.25) (layer F.Cu) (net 4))
 (segment (start 139.446 87.654) (end 139.446 84.074) (width 0.25) (layer F.Cu) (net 4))
 (segment (start 138.747 81.217) (end 139.954 80.01) (width 0.25) (layer F.Cu) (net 13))
 (segment (start 135.445 86.297) (end 135.445 85.915) (width 0.25) (layer F.Cu) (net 13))
 (segment (start 139.954 80.01) (end 140.97 80.01) (width 0.25) (layer F.Cu) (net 13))
 (segment (start 135.445 85.915) (end 138.747 82.613) (width 0.25) (layer F.Cu) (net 13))
 (segment (start 134.366 87.376) (end 135.445 86.297) (width 0.25) (layer F.Cu) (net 13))
 (segment (start 134.054998 87.376) (end 134.366 87.376) (width 0.25) (layer F.Cu) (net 13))
 (segment (start 138.747 82.613) (end 138.747 81.217) (width 0.25) (layer F.Cu) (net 13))
 (segment (start 132.855998 88.575) (end 134.054998 87.376) (width 0.25) (layer F.Cu) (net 13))
 (segment (start 131.75 88.575) (end 132.855998 88.575) (width 0.25) (layer F.Cu) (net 13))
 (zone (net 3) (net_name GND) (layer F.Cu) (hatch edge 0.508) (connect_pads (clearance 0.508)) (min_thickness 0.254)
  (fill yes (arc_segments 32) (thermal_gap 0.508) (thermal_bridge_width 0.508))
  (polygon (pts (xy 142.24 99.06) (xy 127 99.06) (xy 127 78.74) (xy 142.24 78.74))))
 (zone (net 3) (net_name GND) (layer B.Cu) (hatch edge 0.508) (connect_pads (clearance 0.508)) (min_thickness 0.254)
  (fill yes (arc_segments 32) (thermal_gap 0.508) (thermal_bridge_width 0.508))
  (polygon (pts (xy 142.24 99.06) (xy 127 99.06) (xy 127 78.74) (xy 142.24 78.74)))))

